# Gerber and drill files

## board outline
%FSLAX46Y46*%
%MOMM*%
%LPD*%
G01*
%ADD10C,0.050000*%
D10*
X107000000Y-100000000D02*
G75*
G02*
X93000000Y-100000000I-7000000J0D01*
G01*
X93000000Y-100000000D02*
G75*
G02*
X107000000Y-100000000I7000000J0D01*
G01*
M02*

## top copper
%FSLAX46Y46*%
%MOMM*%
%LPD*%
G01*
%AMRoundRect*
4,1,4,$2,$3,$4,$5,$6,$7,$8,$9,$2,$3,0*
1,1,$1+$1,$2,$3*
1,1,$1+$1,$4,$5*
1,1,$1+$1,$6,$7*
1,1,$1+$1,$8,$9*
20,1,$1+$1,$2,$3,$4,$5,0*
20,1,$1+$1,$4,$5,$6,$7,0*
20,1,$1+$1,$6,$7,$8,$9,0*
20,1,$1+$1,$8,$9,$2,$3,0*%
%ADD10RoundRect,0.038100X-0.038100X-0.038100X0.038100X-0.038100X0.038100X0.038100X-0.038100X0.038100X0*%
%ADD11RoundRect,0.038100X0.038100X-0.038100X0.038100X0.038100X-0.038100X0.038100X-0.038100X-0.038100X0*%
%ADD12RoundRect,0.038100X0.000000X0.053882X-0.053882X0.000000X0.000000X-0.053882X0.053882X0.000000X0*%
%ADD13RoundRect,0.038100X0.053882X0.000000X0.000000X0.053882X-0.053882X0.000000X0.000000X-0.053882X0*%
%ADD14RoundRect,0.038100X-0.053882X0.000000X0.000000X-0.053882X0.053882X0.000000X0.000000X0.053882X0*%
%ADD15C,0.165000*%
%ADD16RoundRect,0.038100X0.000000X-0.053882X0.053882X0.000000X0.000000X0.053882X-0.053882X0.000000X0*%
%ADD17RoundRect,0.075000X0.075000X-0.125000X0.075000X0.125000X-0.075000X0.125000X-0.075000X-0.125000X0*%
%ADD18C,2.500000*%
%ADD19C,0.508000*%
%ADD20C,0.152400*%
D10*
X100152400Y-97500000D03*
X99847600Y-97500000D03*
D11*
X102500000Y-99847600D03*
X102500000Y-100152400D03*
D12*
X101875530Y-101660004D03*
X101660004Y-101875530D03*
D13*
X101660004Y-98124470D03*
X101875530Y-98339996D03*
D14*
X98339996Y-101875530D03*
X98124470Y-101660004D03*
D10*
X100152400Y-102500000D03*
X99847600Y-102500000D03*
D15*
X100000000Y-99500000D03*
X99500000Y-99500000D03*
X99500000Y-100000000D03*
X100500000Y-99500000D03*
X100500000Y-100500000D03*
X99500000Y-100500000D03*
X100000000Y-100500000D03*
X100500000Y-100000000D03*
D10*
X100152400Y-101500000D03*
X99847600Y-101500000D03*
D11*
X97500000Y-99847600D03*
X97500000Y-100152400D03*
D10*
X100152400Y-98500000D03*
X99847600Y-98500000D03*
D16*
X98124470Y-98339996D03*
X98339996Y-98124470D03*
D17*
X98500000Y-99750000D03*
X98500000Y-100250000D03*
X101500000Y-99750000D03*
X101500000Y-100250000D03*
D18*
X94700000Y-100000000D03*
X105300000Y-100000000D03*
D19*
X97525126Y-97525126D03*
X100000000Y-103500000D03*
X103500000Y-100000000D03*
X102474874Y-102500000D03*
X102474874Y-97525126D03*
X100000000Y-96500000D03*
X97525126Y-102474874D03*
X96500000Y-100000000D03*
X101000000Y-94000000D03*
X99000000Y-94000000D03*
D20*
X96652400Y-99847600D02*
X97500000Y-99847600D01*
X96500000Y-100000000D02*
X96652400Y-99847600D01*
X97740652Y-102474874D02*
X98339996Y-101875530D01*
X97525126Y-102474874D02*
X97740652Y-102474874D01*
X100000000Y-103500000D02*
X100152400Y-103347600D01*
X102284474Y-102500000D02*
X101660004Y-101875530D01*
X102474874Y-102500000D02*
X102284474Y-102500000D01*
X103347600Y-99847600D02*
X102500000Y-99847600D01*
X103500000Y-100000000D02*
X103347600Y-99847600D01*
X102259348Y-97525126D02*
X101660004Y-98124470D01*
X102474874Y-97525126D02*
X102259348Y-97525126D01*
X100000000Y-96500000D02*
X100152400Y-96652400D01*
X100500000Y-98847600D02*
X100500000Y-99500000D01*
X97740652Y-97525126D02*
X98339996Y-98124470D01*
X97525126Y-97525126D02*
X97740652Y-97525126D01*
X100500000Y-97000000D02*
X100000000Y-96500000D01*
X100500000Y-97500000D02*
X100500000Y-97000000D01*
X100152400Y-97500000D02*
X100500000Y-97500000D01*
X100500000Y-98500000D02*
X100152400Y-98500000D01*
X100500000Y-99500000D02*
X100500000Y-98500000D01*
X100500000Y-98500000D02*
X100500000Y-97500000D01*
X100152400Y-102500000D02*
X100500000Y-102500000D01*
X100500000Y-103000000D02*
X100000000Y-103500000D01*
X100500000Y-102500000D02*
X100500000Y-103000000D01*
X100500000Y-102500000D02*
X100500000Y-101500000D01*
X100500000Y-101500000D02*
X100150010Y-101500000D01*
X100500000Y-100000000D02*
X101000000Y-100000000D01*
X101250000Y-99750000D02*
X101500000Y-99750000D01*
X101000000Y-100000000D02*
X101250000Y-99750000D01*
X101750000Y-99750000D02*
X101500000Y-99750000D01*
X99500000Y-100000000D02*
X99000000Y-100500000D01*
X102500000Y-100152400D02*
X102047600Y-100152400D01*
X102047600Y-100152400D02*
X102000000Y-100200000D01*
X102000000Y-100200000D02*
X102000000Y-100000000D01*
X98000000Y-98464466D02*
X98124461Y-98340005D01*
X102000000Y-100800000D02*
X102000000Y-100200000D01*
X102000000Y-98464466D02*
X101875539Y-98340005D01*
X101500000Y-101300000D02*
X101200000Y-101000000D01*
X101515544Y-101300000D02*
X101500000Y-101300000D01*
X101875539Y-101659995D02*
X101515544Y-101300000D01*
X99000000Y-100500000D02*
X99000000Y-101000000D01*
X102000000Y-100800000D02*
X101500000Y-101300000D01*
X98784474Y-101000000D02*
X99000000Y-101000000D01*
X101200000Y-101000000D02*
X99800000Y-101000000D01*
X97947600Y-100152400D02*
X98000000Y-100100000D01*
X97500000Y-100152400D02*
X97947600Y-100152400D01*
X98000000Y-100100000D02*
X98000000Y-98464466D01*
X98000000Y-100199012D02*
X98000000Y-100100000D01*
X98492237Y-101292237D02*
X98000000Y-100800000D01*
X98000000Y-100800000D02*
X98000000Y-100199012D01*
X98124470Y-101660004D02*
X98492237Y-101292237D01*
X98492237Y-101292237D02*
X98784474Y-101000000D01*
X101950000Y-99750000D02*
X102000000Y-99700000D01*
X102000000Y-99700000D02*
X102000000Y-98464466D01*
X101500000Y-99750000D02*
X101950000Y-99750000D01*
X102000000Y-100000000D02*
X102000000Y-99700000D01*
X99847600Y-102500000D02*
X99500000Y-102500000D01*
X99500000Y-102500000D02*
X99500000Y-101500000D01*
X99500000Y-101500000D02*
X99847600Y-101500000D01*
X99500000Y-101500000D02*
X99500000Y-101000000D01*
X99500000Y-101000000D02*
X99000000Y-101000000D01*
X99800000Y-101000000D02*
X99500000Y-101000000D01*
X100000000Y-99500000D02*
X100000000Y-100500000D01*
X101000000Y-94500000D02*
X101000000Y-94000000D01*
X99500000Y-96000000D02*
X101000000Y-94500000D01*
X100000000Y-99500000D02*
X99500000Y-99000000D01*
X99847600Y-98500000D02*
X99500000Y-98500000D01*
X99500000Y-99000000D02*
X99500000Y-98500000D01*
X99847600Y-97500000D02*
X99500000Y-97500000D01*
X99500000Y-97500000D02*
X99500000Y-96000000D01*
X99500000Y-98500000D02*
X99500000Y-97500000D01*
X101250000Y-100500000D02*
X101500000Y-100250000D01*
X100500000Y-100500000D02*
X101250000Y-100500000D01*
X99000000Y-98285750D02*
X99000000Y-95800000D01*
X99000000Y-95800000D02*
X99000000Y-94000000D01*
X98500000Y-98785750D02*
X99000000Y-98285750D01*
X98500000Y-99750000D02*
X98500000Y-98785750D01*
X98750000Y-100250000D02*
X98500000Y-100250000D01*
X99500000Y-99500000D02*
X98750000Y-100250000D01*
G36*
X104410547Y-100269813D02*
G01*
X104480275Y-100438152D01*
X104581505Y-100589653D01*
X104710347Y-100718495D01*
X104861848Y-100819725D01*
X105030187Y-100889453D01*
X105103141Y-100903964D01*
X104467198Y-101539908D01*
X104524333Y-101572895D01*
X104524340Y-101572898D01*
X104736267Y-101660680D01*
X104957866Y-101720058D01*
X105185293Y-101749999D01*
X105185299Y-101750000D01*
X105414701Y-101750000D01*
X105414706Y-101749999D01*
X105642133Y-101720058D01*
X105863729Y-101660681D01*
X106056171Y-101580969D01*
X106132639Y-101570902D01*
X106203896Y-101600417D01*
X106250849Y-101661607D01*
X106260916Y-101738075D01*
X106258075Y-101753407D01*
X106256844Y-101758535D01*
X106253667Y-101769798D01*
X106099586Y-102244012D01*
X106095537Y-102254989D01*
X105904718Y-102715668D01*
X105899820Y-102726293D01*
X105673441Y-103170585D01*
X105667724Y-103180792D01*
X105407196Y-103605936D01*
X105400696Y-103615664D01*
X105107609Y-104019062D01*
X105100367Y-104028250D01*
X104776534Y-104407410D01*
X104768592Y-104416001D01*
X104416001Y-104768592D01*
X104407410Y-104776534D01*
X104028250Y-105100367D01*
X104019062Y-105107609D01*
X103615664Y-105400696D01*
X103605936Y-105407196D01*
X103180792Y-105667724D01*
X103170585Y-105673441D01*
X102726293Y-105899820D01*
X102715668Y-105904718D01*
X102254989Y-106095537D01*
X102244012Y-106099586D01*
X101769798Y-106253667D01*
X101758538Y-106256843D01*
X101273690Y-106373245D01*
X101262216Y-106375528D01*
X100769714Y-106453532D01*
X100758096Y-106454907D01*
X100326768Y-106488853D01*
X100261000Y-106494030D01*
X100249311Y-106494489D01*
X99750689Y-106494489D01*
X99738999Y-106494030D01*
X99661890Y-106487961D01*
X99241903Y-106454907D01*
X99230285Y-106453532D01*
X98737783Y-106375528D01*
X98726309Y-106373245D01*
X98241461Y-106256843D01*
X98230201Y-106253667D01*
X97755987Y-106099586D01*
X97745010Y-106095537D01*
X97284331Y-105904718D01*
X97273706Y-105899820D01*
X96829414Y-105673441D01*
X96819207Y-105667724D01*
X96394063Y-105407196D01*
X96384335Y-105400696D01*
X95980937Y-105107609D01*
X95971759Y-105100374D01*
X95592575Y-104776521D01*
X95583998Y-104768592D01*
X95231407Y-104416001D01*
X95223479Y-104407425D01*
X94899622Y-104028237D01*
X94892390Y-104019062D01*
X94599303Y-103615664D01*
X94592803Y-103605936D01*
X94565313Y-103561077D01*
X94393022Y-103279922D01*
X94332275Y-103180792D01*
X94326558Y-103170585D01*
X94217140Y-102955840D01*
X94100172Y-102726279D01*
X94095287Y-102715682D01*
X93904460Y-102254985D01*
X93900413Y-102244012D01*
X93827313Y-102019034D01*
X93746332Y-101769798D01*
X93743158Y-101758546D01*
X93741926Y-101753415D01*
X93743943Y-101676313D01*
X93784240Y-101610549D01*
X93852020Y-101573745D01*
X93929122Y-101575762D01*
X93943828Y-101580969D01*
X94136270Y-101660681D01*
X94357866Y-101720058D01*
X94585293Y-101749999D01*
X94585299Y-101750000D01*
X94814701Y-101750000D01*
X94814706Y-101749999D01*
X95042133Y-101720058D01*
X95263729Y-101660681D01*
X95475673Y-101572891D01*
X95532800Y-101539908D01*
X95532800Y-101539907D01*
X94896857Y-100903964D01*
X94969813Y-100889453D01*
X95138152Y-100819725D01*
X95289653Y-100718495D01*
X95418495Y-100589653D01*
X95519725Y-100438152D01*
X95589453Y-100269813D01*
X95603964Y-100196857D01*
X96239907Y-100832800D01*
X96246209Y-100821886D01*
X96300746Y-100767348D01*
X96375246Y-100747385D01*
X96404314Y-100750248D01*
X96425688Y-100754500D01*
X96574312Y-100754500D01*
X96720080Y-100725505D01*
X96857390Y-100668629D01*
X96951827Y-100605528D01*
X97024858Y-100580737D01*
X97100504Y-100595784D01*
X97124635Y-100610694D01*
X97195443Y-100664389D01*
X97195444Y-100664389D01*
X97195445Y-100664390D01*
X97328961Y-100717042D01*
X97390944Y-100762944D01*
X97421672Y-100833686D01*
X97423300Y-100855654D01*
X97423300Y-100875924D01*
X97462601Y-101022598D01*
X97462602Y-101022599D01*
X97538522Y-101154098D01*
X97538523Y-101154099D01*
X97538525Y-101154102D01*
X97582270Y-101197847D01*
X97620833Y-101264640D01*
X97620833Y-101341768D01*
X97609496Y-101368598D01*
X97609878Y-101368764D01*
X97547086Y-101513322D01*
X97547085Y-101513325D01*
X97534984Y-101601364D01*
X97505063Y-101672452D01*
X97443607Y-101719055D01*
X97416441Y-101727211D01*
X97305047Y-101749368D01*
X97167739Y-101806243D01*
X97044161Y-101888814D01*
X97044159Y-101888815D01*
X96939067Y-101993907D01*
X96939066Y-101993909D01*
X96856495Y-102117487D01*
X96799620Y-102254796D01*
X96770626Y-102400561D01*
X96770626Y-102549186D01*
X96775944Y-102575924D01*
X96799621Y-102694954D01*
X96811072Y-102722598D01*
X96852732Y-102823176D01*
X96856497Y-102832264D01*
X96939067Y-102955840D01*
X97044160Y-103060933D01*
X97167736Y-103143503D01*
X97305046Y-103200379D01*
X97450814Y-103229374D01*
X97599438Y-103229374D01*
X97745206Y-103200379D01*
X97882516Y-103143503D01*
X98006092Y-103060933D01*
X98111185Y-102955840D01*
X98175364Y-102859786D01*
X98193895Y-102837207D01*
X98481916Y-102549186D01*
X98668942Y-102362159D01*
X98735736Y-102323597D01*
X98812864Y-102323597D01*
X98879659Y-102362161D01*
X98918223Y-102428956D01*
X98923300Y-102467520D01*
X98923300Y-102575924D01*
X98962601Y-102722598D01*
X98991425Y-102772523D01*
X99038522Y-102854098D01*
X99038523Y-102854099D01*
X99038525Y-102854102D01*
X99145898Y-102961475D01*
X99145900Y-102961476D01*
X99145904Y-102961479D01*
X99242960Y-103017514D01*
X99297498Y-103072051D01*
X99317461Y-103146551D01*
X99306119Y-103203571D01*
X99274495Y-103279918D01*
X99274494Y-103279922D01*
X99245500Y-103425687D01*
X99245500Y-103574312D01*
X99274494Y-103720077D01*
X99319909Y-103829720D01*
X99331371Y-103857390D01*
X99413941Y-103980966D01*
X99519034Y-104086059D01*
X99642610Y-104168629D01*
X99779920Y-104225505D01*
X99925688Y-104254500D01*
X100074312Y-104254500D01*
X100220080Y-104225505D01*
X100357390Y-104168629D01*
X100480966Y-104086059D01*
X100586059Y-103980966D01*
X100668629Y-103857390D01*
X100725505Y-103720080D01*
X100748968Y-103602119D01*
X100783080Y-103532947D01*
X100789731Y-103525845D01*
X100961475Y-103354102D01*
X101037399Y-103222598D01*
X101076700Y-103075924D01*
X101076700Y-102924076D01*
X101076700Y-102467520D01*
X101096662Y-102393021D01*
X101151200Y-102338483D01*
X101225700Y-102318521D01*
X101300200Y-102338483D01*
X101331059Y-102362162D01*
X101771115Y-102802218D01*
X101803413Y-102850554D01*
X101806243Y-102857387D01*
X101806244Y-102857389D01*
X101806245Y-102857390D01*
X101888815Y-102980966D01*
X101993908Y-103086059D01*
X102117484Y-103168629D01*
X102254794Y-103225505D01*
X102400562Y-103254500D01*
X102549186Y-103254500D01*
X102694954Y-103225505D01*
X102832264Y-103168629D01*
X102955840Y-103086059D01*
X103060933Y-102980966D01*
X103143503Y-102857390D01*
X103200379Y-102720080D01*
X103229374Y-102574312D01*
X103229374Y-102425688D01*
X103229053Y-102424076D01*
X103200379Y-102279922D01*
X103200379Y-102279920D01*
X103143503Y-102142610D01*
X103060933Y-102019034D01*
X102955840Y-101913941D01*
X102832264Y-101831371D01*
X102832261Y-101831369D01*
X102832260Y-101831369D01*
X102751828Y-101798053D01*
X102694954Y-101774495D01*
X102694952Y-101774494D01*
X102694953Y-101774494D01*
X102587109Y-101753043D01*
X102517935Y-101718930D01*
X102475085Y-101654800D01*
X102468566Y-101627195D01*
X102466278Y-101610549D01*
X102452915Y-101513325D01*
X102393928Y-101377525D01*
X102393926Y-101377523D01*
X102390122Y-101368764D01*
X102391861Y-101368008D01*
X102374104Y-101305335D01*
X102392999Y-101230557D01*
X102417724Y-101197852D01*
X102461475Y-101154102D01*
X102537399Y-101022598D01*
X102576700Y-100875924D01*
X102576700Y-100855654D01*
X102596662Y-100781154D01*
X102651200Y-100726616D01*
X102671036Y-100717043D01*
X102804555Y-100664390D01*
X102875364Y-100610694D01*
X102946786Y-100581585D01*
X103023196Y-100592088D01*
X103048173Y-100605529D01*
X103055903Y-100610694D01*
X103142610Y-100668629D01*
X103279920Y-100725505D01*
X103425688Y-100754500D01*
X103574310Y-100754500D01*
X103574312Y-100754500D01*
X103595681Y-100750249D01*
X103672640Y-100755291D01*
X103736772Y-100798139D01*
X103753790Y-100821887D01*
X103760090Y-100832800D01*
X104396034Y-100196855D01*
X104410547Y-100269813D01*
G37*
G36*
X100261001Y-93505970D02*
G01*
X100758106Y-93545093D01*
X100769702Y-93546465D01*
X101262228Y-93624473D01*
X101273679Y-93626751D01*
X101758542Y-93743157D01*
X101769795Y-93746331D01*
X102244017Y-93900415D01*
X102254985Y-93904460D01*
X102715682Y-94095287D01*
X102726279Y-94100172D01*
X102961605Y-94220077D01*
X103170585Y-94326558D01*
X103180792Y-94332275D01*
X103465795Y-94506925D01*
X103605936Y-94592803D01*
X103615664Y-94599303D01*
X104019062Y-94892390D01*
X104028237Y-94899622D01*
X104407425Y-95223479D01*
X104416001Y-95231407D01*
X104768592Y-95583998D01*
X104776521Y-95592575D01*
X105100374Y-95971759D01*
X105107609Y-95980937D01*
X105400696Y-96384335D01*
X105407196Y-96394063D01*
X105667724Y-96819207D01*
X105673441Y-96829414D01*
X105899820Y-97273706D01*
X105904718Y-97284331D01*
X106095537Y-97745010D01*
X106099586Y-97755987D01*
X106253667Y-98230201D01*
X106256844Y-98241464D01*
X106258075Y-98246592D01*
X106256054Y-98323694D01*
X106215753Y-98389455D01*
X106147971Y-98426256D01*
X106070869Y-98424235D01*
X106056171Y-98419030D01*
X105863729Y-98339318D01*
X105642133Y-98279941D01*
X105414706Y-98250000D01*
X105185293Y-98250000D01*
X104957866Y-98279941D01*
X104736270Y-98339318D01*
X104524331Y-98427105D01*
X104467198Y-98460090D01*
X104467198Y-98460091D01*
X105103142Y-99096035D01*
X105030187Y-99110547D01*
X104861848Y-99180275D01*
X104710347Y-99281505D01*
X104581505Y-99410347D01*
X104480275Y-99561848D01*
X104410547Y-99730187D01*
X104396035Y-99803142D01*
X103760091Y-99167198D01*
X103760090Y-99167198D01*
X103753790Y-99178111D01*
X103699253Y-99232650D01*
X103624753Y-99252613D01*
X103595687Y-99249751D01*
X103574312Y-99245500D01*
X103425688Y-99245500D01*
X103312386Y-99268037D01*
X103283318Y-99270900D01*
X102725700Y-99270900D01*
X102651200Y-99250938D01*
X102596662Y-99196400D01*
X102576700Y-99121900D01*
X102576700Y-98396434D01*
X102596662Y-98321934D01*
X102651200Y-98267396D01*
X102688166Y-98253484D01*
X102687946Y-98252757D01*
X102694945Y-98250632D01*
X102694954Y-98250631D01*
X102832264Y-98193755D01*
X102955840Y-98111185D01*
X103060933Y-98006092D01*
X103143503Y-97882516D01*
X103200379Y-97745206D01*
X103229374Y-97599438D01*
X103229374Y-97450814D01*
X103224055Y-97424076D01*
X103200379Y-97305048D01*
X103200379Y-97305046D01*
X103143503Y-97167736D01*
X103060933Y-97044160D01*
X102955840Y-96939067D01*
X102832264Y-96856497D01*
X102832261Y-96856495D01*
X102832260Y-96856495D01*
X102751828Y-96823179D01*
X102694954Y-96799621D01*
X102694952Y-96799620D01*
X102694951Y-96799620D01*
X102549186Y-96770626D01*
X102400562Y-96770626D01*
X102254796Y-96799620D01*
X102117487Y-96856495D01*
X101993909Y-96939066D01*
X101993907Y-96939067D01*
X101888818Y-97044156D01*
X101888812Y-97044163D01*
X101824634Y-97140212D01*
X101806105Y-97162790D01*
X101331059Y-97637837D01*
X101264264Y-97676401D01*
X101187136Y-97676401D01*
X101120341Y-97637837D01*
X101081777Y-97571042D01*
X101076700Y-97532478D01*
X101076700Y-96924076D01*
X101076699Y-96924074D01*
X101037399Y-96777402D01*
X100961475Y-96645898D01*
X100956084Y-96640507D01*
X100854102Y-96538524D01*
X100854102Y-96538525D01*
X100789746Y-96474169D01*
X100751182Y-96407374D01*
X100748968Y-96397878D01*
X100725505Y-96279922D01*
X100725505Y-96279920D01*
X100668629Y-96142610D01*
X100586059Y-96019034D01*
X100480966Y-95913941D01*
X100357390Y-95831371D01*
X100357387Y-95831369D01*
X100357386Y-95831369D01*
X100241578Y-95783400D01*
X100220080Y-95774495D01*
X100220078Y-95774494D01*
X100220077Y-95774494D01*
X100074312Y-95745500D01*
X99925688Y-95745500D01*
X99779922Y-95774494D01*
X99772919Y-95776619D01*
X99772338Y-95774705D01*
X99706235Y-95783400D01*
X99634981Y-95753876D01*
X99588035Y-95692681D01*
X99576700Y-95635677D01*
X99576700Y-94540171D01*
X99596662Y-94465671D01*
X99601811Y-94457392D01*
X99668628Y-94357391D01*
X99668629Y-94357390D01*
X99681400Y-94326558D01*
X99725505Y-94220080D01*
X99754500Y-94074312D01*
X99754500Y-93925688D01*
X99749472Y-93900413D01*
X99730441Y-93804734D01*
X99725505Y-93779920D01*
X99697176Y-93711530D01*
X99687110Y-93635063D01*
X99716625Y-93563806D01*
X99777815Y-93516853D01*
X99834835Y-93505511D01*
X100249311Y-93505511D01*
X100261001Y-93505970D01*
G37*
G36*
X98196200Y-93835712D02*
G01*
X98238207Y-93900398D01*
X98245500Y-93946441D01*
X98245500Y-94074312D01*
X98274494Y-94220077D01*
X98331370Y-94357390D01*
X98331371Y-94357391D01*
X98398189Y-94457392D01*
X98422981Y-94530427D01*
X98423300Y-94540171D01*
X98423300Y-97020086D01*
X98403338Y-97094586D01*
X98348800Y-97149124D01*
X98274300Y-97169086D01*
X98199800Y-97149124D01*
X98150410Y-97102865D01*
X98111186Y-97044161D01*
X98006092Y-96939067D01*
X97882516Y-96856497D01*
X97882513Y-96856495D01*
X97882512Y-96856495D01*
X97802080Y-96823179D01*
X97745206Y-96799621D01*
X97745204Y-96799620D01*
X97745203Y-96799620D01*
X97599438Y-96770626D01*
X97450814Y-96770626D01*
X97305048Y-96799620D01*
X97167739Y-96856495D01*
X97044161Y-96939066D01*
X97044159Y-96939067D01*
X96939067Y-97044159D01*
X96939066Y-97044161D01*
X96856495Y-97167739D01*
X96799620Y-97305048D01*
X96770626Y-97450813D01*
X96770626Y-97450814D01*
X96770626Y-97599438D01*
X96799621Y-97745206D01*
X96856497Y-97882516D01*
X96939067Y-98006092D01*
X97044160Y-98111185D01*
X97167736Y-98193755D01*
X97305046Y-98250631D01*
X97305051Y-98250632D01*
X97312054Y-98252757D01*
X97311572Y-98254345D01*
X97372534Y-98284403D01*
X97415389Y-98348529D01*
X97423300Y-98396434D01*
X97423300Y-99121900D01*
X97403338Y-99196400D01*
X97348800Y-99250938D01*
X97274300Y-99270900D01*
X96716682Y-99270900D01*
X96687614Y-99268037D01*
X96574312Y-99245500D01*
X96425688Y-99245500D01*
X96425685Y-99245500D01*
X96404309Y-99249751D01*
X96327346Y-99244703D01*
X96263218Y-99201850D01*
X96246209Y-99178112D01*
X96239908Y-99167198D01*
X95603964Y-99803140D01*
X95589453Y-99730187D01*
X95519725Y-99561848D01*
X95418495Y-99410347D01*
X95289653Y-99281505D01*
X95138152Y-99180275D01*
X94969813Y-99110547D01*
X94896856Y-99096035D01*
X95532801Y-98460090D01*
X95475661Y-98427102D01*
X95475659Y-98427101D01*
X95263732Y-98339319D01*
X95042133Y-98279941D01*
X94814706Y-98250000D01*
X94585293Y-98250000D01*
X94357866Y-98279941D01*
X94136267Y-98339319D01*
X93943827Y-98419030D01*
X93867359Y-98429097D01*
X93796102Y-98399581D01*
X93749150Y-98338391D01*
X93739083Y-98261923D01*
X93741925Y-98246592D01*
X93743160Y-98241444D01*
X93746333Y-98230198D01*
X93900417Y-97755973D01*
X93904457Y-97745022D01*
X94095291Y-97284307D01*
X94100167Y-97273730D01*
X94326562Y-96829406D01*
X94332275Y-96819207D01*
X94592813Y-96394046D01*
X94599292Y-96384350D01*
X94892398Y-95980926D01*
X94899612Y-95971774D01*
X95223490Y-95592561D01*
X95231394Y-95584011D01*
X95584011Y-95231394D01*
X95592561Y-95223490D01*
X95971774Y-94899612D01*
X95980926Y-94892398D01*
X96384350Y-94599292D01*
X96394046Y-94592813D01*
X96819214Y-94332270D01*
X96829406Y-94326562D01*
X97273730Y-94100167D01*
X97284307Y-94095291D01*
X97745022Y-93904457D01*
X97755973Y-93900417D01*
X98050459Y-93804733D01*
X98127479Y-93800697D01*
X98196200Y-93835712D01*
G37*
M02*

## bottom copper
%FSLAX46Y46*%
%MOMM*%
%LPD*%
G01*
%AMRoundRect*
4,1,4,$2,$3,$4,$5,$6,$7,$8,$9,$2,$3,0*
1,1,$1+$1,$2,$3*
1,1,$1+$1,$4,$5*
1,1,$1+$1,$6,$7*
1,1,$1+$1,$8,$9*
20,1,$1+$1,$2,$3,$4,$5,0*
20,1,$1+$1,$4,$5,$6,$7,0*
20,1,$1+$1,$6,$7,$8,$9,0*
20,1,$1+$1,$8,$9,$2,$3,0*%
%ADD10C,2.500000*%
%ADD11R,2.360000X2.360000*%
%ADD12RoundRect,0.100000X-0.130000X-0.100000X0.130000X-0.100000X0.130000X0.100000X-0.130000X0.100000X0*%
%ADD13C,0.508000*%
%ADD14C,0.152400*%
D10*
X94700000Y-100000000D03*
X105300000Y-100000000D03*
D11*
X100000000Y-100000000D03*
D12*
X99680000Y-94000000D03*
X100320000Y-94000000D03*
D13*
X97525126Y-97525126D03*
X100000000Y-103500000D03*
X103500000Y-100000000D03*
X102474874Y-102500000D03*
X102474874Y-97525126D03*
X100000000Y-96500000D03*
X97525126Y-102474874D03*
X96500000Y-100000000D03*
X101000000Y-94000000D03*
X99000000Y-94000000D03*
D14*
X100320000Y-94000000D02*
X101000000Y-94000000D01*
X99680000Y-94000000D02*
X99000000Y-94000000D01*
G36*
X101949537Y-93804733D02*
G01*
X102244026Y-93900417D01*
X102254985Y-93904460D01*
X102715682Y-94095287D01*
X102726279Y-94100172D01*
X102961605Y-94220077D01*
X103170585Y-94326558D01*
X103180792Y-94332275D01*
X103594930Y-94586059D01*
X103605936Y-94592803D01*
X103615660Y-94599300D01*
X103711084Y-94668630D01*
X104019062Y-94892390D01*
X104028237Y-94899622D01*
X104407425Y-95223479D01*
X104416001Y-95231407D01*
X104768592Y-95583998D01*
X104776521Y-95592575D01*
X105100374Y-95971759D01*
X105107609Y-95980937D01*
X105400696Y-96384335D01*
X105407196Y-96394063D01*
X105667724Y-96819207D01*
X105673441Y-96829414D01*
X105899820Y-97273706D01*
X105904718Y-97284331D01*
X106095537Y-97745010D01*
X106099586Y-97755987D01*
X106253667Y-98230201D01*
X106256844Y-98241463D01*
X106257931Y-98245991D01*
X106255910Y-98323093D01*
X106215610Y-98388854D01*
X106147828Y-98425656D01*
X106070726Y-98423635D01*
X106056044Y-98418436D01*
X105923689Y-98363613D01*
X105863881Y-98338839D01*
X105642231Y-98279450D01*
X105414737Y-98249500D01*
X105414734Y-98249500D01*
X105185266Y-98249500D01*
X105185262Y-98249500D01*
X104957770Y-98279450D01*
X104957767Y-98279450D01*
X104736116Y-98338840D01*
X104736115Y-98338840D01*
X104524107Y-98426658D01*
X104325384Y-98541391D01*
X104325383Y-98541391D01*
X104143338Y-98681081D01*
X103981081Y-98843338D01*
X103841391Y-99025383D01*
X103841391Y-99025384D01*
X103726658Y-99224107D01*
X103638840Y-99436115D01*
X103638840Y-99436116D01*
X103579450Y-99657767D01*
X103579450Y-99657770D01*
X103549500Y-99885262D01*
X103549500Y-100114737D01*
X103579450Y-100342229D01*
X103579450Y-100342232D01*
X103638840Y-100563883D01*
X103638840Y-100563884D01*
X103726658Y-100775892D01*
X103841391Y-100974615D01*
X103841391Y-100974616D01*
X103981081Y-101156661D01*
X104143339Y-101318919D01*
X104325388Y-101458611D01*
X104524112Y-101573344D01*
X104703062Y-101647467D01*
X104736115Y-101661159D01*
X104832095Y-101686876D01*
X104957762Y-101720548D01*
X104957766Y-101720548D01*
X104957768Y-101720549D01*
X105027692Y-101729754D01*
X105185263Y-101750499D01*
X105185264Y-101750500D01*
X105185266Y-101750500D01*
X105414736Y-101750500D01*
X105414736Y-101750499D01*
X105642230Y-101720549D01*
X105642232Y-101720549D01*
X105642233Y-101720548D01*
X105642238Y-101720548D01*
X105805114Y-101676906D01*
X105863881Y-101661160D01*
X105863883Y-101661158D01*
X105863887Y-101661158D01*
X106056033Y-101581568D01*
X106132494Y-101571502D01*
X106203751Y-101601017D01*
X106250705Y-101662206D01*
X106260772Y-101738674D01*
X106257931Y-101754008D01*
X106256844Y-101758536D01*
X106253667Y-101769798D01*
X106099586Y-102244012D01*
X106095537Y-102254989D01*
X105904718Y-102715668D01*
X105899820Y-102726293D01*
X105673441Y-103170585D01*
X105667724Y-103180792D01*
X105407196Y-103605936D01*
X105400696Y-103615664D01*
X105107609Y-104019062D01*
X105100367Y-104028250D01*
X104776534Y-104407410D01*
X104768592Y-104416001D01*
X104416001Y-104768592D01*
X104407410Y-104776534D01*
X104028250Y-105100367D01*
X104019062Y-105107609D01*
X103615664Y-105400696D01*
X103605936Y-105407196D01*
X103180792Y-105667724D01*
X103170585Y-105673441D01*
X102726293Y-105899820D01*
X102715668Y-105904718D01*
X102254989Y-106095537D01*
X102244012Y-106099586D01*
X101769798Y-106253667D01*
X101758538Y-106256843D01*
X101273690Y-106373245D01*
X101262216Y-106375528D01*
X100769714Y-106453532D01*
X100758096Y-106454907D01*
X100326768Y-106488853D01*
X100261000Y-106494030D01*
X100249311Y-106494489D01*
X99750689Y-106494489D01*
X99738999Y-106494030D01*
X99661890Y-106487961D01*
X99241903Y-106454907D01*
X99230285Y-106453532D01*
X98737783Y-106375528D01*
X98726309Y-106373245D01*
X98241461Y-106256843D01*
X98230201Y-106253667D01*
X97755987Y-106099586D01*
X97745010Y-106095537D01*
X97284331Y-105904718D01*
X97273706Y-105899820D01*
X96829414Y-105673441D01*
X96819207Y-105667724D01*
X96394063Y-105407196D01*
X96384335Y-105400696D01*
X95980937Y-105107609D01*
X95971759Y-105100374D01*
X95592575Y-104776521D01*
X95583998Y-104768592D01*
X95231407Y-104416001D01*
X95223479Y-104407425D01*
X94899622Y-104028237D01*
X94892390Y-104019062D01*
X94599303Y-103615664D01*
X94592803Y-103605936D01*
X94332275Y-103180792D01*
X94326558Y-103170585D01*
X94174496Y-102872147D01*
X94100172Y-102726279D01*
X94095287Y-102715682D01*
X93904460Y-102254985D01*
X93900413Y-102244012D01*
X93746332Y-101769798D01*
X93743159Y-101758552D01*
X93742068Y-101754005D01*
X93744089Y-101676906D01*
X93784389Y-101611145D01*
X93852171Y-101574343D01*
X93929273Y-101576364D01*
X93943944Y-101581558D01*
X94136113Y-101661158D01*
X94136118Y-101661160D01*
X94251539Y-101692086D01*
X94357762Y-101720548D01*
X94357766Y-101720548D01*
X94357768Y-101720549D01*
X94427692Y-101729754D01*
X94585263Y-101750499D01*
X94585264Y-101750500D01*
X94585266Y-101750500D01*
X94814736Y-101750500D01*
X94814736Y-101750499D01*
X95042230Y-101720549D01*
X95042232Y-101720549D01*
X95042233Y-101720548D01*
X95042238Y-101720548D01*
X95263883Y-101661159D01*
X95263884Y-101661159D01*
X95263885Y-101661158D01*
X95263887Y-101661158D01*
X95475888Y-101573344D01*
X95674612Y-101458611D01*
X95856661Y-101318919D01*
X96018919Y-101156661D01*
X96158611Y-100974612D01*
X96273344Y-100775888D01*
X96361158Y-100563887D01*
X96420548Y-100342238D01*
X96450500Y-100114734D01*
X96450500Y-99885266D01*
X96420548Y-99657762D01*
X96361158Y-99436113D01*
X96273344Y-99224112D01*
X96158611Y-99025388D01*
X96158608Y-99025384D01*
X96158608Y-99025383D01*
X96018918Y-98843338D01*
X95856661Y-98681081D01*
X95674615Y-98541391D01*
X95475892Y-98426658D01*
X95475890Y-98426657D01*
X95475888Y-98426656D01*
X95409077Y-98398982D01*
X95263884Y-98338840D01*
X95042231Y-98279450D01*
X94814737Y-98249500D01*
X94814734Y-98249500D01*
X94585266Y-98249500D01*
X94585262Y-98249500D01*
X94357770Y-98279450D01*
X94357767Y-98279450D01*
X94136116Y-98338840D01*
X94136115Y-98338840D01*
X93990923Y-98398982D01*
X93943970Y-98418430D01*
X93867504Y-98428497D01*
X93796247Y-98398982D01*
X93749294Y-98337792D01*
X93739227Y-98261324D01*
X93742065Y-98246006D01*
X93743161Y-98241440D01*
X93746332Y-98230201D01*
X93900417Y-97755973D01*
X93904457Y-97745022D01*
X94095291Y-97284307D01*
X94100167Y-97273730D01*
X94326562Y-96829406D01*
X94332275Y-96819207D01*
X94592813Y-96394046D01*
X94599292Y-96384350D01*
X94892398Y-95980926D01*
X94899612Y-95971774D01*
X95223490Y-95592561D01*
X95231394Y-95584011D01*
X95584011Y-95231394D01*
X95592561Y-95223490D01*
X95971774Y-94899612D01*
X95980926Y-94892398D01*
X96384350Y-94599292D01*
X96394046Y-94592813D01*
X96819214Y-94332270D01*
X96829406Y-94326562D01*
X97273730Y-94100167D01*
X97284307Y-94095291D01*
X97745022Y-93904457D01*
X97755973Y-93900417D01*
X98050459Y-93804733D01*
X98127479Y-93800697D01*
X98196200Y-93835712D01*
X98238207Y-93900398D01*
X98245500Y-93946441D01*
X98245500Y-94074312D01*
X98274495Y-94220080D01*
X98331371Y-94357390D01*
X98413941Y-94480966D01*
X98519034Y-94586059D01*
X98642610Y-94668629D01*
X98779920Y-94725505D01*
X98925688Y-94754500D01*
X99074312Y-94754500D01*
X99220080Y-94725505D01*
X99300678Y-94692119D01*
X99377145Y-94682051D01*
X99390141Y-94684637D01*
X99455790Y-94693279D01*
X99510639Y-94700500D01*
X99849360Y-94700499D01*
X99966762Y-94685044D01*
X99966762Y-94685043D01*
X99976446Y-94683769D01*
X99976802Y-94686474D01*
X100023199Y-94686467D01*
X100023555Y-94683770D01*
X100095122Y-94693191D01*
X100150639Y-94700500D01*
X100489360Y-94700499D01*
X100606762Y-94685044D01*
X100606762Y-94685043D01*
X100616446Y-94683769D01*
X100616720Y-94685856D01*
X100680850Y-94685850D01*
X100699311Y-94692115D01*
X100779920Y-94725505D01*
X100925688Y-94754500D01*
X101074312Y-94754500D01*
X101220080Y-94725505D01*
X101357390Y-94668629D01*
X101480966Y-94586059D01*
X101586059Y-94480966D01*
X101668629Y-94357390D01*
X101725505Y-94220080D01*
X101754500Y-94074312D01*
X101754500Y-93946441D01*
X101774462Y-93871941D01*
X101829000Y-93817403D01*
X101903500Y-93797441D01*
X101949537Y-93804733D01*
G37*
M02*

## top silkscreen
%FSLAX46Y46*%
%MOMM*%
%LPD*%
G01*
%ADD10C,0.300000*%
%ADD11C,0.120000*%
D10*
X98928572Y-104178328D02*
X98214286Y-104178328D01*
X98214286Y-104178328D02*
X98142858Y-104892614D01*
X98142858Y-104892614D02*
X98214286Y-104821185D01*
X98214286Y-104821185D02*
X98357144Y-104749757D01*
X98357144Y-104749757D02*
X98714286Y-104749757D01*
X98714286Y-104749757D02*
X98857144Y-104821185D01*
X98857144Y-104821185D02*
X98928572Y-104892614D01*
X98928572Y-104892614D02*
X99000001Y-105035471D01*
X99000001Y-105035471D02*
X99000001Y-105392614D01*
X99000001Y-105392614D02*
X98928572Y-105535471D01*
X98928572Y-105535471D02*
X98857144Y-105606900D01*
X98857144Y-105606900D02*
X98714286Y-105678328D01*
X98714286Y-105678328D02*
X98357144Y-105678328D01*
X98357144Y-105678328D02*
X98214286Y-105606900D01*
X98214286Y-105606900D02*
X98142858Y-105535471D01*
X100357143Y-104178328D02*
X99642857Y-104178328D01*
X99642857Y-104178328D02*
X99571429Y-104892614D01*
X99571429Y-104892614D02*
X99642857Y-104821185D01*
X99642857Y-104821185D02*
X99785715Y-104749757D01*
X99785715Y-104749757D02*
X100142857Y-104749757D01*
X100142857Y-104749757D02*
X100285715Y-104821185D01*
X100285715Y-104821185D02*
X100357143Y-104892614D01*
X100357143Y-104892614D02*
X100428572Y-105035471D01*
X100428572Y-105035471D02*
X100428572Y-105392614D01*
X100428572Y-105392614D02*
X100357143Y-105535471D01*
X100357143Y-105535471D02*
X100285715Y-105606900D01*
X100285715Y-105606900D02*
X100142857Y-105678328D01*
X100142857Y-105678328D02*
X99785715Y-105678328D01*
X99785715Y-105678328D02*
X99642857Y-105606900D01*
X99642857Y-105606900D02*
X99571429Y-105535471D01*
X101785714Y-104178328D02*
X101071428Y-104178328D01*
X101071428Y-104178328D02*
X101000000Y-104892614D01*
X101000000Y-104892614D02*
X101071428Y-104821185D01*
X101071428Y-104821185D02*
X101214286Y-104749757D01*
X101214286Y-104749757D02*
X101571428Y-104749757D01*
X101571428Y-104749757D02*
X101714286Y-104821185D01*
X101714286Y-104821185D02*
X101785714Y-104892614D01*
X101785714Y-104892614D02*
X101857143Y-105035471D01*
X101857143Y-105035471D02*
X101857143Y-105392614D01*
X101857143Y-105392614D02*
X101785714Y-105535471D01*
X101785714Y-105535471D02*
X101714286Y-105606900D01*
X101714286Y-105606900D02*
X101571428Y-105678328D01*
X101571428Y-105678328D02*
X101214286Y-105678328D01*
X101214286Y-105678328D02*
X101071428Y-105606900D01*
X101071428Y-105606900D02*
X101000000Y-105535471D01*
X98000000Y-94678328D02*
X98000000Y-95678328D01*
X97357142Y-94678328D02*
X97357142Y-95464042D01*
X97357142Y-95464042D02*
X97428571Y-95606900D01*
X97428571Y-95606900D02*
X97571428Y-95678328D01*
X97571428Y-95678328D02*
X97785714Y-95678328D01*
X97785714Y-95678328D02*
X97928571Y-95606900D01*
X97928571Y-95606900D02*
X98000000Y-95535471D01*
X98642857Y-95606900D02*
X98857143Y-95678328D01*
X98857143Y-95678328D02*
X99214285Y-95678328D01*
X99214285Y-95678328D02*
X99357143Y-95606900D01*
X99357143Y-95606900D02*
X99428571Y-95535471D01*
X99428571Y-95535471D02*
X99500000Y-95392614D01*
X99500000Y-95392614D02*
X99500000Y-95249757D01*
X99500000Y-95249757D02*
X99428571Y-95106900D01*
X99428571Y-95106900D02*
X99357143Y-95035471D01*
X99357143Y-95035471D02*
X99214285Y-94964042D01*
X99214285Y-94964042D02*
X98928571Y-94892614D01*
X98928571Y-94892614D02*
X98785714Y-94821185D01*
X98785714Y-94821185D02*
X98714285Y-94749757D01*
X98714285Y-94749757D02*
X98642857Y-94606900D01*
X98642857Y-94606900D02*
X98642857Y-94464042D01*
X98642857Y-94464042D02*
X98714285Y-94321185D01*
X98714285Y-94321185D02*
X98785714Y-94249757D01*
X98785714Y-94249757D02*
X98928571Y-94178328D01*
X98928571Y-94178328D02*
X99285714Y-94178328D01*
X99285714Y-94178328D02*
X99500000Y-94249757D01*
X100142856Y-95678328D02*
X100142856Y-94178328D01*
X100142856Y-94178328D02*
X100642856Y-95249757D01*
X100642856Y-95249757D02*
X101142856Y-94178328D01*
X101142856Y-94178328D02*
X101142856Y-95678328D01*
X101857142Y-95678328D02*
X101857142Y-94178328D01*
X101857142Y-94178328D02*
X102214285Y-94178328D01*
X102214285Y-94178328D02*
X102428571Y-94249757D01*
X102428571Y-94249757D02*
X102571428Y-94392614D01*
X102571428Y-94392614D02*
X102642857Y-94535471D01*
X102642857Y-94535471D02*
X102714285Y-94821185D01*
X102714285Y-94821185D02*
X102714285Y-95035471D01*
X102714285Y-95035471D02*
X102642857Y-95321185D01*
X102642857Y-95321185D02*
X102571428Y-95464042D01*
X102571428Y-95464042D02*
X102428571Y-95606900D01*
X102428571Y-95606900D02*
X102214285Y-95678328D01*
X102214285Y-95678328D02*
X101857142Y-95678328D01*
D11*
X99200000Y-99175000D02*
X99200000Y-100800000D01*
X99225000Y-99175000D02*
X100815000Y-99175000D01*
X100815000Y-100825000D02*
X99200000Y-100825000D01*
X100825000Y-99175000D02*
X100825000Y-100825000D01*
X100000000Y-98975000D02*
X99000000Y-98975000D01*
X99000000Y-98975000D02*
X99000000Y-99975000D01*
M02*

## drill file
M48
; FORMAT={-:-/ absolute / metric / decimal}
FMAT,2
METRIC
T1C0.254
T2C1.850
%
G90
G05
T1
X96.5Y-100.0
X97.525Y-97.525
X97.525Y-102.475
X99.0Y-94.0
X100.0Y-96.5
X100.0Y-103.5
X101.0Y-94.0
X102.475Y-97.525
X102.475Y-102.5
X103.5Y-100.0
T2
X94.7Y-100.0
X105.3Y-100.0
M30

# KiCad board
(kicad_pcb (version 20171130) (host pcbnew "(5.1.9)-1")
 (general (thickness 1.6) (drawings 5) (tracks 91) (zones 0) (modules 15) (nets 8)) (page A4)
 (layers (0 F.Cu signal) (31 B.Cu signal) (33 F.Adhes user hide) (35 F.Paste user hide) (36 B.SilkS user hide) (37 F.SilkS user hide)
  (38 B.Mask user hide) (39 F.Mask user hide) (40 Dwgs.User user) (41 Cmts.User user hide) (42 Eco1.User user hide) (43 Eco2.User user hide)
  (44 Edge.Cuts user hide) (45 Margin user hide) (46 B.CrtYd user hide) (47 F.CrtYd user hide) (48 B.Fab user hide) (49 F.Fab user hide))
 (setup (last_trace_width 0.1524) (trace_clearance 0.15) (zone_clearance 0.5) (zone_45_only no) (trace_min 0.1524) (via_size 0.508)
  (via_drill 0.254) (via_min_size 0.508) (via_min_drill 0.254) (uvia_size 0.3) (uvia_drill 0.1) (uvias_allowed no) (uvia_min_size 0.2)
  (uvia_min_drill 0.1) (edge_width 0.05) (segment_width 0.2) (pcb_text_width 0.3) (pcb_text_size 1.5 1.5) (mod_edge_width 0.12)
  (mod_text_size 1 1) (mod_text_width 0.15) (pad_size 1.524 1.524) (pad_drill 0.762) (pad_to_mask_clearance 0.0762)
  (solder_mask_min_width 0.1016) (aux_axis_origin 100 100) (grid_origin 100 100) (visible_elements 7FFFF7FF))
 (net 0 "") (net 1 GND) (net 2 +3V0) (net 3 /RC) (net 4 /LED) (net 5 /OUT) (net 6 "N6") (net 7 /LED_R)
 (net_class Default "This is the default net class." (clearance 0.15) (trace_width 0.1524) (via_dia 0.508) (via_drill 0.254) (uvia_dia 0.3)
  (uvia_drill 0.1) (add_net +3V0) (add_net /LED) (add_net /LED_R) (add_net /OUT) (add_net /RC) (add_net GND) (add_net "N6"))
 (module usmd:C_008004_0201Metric (layer F.Cu) (at 100 97.5)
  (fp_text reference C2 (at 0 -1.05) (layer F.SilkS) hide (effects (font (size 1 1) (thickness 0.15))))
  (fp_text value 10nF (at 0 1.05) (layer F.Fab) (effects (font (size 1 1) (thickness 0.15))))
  (pad 2 smd roundrect (at 0.1524 0) (size 0.1524 0.1524) (layers F.Cu F.Mask) (roundrect_rratio 0.25) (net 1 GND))
  (pad 1 smd roundrect (at -0.1524 0) (size 0.1524 0.1524) (layers F.Cu F.Paste F.Mask) (roundrect_rratio 0.25) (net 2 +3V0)))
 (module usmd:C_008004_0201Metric (layer F.Cu) (at 102.5 100 90)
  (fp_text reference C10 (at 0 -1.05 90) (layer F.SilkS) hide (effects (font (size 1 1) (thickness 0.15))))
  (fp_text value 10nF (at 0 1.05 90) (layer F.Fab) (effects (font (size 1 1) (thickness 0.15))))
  (pad 2 smd roundrect (at 0.1524 0 90) (size 0.1524 0.1524) (layers F.Cu F.Mask) (roundrect_rratio 0.25) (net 1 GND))
  (pad 1 smd roundrect (at -0.1524 0 90) (size 0.1524 0.1524) (layers F.Cu F.Paste F.Mask) (roundrect_rratio 0.25) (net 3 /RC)))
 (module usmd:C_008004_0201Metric (layer F.Cu) (at 101.767767 101.767767 225)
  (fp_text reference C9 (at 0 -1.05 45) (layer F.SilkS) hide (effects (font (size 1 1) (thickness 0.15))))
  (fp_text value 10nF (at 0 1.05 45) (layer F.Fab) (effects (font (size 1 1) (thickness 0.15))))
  (pad 1 smd roundrect (at -0.1524 0 225) (size 0.1524 0.1524) (layers F.Cu F.Paste F.Mask) (roundrect_rratio 0.25) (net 3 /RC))
  (pad 2 smd roundrect (at 0.1524 0 225) (size 0.1524 0.1524) (layers F.Cu F.Mask) (roundrect_rratio 0.25) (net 1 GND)))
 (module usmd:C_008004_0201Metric (layer F.Cu) (at 101.767767 98.232233 135)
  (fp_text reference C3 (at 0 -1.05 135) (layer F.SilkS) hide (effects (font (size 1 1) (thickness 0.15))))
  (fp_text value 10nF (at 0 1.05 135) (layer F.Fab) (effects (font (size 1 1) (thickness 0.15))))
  (pad 2 smd roundrect (at 0.1524 0 135) (size 0.1524 0.1524) (layers F.Cu F.Mask) (roundrect_rratio 0.25) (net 1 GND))
  (pad 1 smd roundrect (at -0.1524 0 135) (size 0.1524 0.1524) (layers F.Cu F.Paste F.Mask) (roundrect_rratio 0.25) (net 3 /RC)))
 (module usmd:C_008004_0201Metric (layer F.Cu) (at 98.232233 101.767767 315)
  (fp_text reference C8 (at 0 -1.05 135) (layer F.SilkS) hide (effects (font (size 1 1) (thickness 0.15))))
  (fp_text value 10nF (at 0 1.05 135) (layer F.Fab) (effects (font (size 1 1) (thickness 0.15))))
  (pad 2 smd roundrect (at 0.1524 0 315) (size 0.1524 0.1524) (layers F.Cu F.Mask) (roundrect_rratio 0.25) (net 1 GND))
  (pad 1 smd roundrect (at -0.1524 0 315) (size 0.1524 0.1524) (layers F.Cu F.Paste F.Mask) (roundrect_rratio 0.25) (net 3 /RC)))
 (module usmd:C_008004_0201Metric (layer F.Cu) (at 100 102.5)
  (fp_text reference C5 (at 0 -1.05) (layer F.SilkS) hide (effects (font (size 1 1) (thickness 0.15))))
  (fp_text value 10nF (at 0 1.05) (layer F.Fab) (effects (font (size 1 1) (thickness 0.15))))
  (pad 2 smd roundrect (at 0.1524 0) (size 0.1524 0.1524) (layers F.Cu F.Mask) (roundrect_rratio 0.25) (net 1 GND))
  (pad 1 smd roundrect (at -0.1524 0) (size 0.1524 0.1524) (layers F.Cu F.Paste F.Mask) (roundrect_rratio 0.25) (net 3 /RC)))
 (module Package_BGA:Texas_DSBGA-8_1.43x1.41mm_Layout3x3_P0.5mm (layer F.Cu) (at 100 100) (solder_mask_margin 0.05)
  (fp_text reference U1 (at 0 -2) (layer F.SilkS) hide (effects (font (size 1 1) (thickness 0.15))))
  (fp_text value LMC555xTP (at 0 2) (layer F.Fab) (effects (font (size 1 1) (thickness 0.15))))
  (fp_line (start -0.8 -0.825) (end -0.8 0.8) (layer F.SilkS) (width 0.12))
  (fp_line (start -0.775 -0.825) (end 0.815 -0.825) (layer F.SilkS) (width 0.12))
  (fp_line (start 0.815 0.825) (end -0.8 0.825) (layer F.SilkS) (width 0.12))
  (fp_line (start 0.825 -0.825) (end 0.825 0.825) (layer F.SilkS) (width 0.12))
  (fp_line (start 0 -1.025) (end -1 -1.025) (layer F.SilkS) (width 0.12))
  (fp_line (start -1 -1.025) (end -1 -0.025) (layer F.SilkS) (width 0.12))
  (pad "" smd rect (at 0.5 0.5) (size 0.3 0.3) (layers F.Paste)) (pad "" smd rect (at 0 0.5) (size 0.3 0.3) (layers F.Paste))
  (pad "" smd rect (at -0.5 0.5) (size 0.3 0.3) (layers F.Paste)) (pad "" smd rect (at 0.5 0) (size 0.3 0.3) (layers F.Paste))
  (pad "" smd rect (at -0.5 0) (size 0.3 0.3) (layers F.Paste))
  (pad "" smd rect (at 0.5 -0.5) (size 0.3 0.3) (layers F.Paste))
  (pad "" smd rect (at 0 -0.5) (size 0.3 0.3) (layers F.Paste))
  (pad "" smd rect (at -0.5 -0.5) (size 0.3 0.3) (layers F.Paste))
  (pad A2 smd circle (at 0 -0.5) (size 0.165 0.165) (layers F.Cu F.Mask) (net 2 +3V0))
  (pad A1 smd circle (at -0.5 -0.5) (size 0.165 0.165) (layers F.Cu F.Mask) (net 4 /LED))
  (pad B1 smd circle (at -0.5 0) (size 0.165 0.165) (layers F.Cu F.Mask) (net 3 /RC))
  (pad A3 smd circle (at 0.5 -0.5) (size 0.165 0.165) (layers F.Cu F.Mask) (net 1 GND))
  (pad C3 smd circle (at 0.5 0.5) (size 0.165 0.165) (layers F.Cu F.Mask) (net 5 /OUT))
  (pad C1 smd circle (at -0.5 0.5) (size 0.165 0.165) (layers F.Cu F.Mask) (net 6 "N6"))
  (pad C2 smd circle (at 0 0.5) (size 0.165 0.165) (layers F.Cu F.Mask) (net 2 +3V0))
  (pad B3 smd circle (at 0.5 0) (size 0.165 0.165) (layers F.Cu F.Paste F.Mask) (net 3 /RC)))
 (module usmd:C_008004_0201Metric (layer F.Cu) (at 100 101.5)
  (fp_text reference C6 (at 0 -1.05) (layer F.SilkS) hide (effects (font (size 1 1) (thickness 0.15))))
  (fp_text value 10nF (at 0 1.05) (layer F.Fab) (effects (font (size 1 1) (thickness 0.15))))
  (pad 2 smd roundrect (at 0.1524 0) (size 0.1524 0.1524) (layers F.Cu F.Mask) (roundrect_rratio 0.25) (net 1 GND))
  (pad 1 smd roundrect (at -0.1524 0) (size 0.1524 0.1524) (layers F.Cu F.Paste F.Mask) (roundrect_rratio 0.25) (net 3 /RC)))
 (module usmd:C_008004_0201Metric (layer F.Cu) (at 97.5 100 90)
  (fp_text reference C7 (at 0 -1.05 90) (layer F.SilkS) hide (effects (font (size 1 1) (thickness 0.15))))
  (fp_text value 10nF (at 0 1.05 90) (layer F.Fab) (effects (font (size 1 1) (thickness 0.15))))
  (pad 2 smd roundrect (at 0.1524 0 90) (size 0.1524 0.1524) (layers F.Cu F.Mask) (roundrect_rratio 0.25) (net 1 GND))
  (pad 1 smd roundrect (at -0.1524 0 90) (size 0.1524 0.1524) (layers F.Cu F.Paste F.Mask) (roundrect_rratio 0.25) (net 3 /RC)))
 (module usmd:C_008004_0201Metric (layer F.Cu) (at 100 98.5)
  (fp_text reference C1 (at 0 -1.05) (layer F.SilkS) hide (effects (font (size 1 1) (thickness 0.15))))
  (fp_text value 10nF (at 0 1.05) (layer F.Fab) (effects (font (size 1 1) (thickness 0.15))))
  (pad 2 smd roundrect (at 0.1524 0) (size 0.1524 0.1524) (layers F.Cu F.Mask) (roundrect_rratio 0.25) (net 1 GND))
  (pad 1 smd roundrect (at -0.1524 0) (size 0.1524 0.1524) (layers F.Cu F.Paste F.Mask) (roundrect_rratio 0.25) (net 2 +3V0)))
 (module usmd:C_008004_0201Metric (layer F.Cu) (at 98.232233 98.232233 45)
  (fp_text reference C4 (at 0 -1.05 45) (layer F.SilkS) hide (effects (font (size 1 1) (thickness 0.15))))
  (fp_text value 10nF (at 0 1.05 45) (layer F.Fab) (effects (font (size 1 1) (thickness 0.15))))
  (pad 1 smd roundrect (at -0.1524 0 45) (size 0.1524 0.1524) (layers F.Cu F.Paste F.Mask) (roundrect_rratio 0.25) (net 3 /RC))
  (pad 2 smd roundrect (at 0.1524 0 45) (size 0.1524 0.1524) (layers F.Cu F.Mask) (roundrect_rratio 0.25) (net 1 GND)))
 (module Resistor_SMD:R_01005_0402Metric (layer F.Cu) (at 98.5 100 90)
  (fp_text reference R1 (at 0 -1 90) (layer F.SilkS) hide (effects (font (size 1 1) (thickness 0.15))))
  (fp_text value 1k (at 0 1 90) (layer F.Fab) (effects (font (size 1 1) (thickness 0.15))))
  (pad 2 smd roundrect (at 0.25 0 90) (size 0.4 0.3) (layers F.Cu F.Mask) (roundrect_rratio 0.25) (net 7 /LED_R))
  (pad 1 smd roundrect (at -0.25 0 90) (size 0.4 0.3) (layers F.Cu F.Mask) (roundrect_rratio 0.25) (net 4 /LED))
  (pad "" smd roundrect (at 0.275 0 90) (size 0.27 0.27) (layers F.Paste) (roundrect_rratio 0.25))
  (pad "" smd roundrect (at -0.275 0 90) (size 0.27 0.27) (layers F.Paste) (roundrect_rratio 0.25)))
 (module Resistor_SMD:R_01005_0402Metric (layer F.Cu) (at 101.5 100 90)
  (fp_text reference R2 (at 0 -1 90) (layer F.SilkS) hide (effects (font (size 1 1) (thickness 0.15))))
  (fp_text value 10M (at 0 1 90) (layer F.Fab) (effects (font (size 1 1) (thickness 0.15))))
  (pad 2 smd roundrect (at 0.25 0 90) (size 0.4 0.3) (layers F.Cu F.Mask) (roundrect_rratio 0.25) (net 3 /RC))
  (pad 1 smd roundrect (at -0.25 0 90) (size 0.4 0.3) (layers F.Cu F.Mask) (roundrect_rratio 0.25) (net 5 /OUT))
  (pad "" smd roundrect (at 0.275 0 90) (size 0.27 0.27) (layers F.Paste) (roundrect_rratio 0.25))
  (pad "" smd roundrect (at -0.275 0 90) (size 0.27 0.27) (layers F.Paste) (roundrect_rratio 0.25)))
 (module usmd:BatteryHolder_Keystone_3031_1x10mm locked (layer B.Cu) (at 100 100)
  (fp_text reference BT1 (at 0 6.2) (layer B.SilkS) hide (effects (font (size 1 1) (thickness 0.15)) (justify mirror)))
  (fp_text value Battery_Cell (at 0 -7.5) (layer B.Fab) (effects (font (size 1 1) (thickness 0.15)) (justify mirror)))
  (pad 1 thru_hole circle (at -5.3 0) (size 2.5 2.5) (drill 1.85) (layers *.Cu *.Mask) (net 2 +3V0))
  (pad 1 thru_hole circle (at 5.3 0) (size 2.5 2.5) (drill 1.85) (layers *.Cu *.Mask) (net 2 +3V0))
  (pad 2 smd rect (at 0 0) (size 2.36 2.36) (layers B.Cu B.Mask) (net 1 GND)))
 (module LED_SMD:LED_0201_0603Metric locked (layer B.Cu) (at 100 94)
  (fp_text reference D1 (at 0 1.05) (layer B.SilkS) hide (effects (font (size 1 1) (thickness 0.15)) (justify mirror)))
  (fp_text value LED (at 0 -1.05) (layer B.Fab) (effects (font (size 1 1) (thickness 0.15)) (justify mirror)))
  (pad "" smd roundrect (at -0.345 0) (size 0.318 0.36) (layers B.Paste) (roundrect_rratio 0.25))
  (pad "" smd roundrect (at 0.345 0) (size 0.318 0.36) (layers B.Paste) (roundrect_rratio 0.25))
  (pad 1 smd roundrect (at -0.32 0) (size 0.46 0.4) (layers B.Cu B.Mask) (roundrect_rratio 0.25) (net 7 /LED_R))
  (pad 2 smd roundrect (at 0.32 0) (size 0.46 0.4) (layers B.Cu B.Mask) (roundrect_rratio 0.25) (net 2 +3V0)))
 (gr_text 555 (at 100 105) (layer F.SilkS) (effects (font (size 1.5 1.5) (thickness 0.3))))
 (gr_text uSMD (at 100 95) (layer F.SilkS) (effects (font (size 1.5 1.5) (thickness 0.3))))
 (gr_circle (center 100 100) (end 107 100) (layer Edge.Cuts) (width 0.05))
 (via (at 97.525126 97.525126) (size 0.508) (drill 0.254) (layers F.Cu B.Cu) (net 1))
 (via (at 100 103.5) (size 0.508) (drill 0.254) (layers F.Cu B.Cu) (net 1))
 (via (at 103.5 100) (size 0.508) (drill 0.254) (layers F.Cu B.Cu) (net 1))
 (via (at 102.474874 102.5) (size 0.508) (drill 0.254) (layers F.Cu B.Cu) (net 1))
 (via (at 102.474874 97.525126) (size 0.508) (drill 0.254) (layers F.Cu B.Cu) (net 1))
 (via (at 100 96.5) (size 0.508) (drill 0.254) (layers F.Cu B.Cu) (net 1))
 (via (at 97.525126 102.474874) (size 0.508) (drill 0.254) (layers F.Cu B.Cu) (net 1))
 (via (at 96.5 100) (size 0.508) (drill 0.254) (layers F.Cu B.Cu) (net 1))
 (segment (start 96.6524 99.8476) (end 97.5 99.8476) (width 0.1524) (layer F.Cu) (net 1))
 (segment (start 96.5 100) (end 96.6524 99.8476) (width 0.1524) (layer F.Cu) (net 1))
 (segment (start 97.740652 102.474874) (end 98.339996 101.87553) (width 0.1524) (layer F.Cu) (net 1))
 (segment (start 97.525126 102.474874) (end 97.740652 102.474874) (width 0.1524) (layer F.Cu) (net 1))
 (segment (start 100 103.5) (end 100.1524 103.3476) (width 0.1524) (layer F.Cu) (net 1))
 (segment (start 102.284474 102.5) (end 101.660004 101.87553) (width 0.1524) (layer F.Cu) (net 1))
 (segment (start 102.474874 102.5) (end 102.284474 102.5) (width 0.1524) (layer F.Cu) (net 1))
 (segment (start 103.3476 99.8476) (end 102.5 99.8476) (width 0.1524) (layer F.Cu) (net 1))
 (segment (start 103.5 100) (end 103.3476 99.8476) (width 0.1524) (layer F.Cu) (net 1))
 (segment (start 102.259348 97.525126) (end 101.660004 98.12447) (width 0.1524) (layer F.Cu) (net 1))
 (segment (start 102.474874 97.525126) (end 102.259348 97.525126) (width 0.1524) (layer F.Cu) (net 1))
 (segment (start 100 96.5) (end 100.1524 96.6524) (width 0.1524) (layer F.Cu) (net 1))
 (segment (start 100.5 98.8476) (end 100.5 99.5) (width 0.1524) (layer F.Cu) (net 1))
 (segment (start 97.740652 97.525126) (end 98.339996 98.12447) (width 0.1524) (layer F.Cu) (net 1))
 (segment (start 97.525126 97.525126) (end 97.740652 97.525126) (width 0.1524) (layer F.Cu) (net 1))
 (segment (start 100.5 97) (end 100 96.5) (width 0.1524) (layer F.Cu) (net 1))
 (segment (start 100.5 97.5) (end 100.5 97) (width 0.1524) (layer F.Cu) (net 1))
 (segment (start 100.1524 97.5) (end 100.5 97.5) (width 0.1524) (layer F.Cu) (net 1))
 (segment (start 100.5 98.5) (end 100.1524 98.5) (width 0.1524) (layer F.Cu) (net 1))
 (segment (start 100.5 99.5) (end 100.5 98.5) (width 0.1524) (layer F.Cu) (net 1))
 (segment (start 100.5 98.5) (end 100.5 97.5) (width 0.1524) (layer F.Cu) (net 1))
 (segment (start 100.1524 102.5) (end 100.5 102.5) (width 0.1524) (layer F.Cu) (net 1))
 (segment (start 100.5 103) (end 100 103.5) (width 0.1524) (layer F.Cu) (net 1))
 (segment (start 100.5 102.5) (end 100.5 103) (width 0.1524) (layer F.Cu) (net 1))
 (segment (start 100.5 102.5) (end 100.5 101.5) (width 0.1524) (layer F.Cu) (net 1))
 (segment (start 100.5 101.5) (end 100.15001 101.5) (width 0.1524) (layer F.Cu) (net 1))
 (segment (start 100.5 100) (end 101 100) (width 0.1524) (layer F.Cu) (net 3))
 (segment (start 101.25 99.75) (end 101.5 99.75) (width 0.1524) (layer F.Cu) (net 3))
 (segment (start 101 100) (end 101.25 99.75) (width 0.1524) (layer F.Cu) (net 3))
 (segment (start 101.75 99.75) (end 101.5 99.75) (width 0.1524) (layer F.Cu) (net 3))
 (segment (start 99.5 100) (end 99 100.5) (width 0.1524) (layer F.Cu) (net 3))
 (segment (start 102.5 100.1524) (end 102.0476 100.1524) (width 0.1524) (layer F.Cu) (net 3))
 (segment (start 102.0476 100.1524) (end 102 100.2) (width 0.1524) (layer F.Cu) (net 3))
 (segment (start 102 100.2) (end 102 100) (width 0.1524) (layer F.Cu) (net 3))
 (segment (start 98 98.464466) (end 98.124461 98.340005) (width 0.1524) (layer F.Cu) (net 3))
 (segment (start 102 100.8) (end 102 100.2) (width 0.1524) (layer F.Cu) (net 3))
 (segment (start 102 98.464466) (end 101.875539 98.340005) (width 0.1524) (layer F.Cu) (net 3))
 (segment (start 101.5 101.3) (end 101.2 101) (width 0.1524) (layer F.Cu) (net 3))
 (segment (start 101.515544 101.3) (end 101.5 101.3) (width 0.1524) (layer F.Cu) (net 3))
 (segment (start 101.875539 101.659995) (end 101.515544 101.3) (width 0.1524) (layer F.Cu) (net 3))
 (segment (start 99 100.5) (end 99 101) (width 0.1524) (layer F.Cu) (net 3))
 (segment (start 102 100.8) (end 101.5 101.3) (width 0.1524) (layer F.Cu) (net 3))
 (segment (start 98.784474 101) (end 99 101) (width 0.1524) (layer F.Cu) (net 3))
 (segment (start 101.2 101) (end 99.8 101) (width 0.1524) (layer F.Cu) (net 3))
 (segment (start 97.9476 100.1524) (end 98 100.1) (width 0.1524) (layer F.Cu) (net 3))
 (segment (start 97.5 100.1524) (end 97.9476 100.1524) (width 0.1524) (layer F.Cu) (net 3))
 (segment (start 98 100.1) (end 98 98.464466) (width 0.1524) (layer F.Cu) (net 3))
 (segment (start 98 100.199012) (end 98 100.1) (width 0.1524) (layer F.Cu) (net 3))
 (segment (start 98.492237 101.292237) (end 98 100.8) (width 0.1524) (layer F.Cu) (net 3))
 (segment (start 98 100.8) (end 98 100.199012) (width 0.1524) (layer F.Cu) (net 3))
 (segment (start 98.12447 101.660004) (end 98.492237 101.292237) (width 0.1524) (layer F.Cu) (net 3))
 (segment (start 98.492237 101.292237) (end 98.784474 101) (width 0.1524) (layer F.Cu) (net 3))
 (segment (start 101.95 99.75) (end 102 99.7) (width 0.1524) (layer F.Cu) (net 3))
 (segment (start 102 99.7) (end 102 98.464466) (width 0.1524) (layer F.Cu) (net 3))
 (segment (start 101.5 99.75) (end 101.95 99.75) (width 0.1524) (layer F.Cu) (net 3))
 (segment (start 102 100) (end 102 99.7) (width 0.1524) (layer F.Cu) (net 3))
 (segment (start 99.8476 102.5) (end 99.5 102.5) (width 0.1524) (layer F.Cu) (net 3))
 (segment (start 99.5 102.5) (end 99.5 101.5) (width 0.1524) (layer F.Cu) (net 3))
 (segment (start 99.5 101.5) (end 99.8476 101.5) (width 0.1524) (layer F.Cu) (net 3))
 (segment (start 99.5 101.5) (end 99.5 101) (width 0.1524) (layer F.Cu) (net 3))
 (segment (start 99.5 101) (end 99 101) (width 0.1524) (layer F.Cu) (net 3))
 (segment (start 99.8 101) (end 99.5 101) (width 0.1524) (layer F.Cu) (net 3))
 (segment (start 100 99.5) (end 100 100.5) (width 0.1524) (layer F.Cu) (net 2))
 (segment (start 100.32 94) (end 101 94) (width 0.1524) (layer B.Cu) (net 2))
 (via (at 101 94) (size 0.508) (drill 0.254) (layers F.Cu B.Cu) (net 2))
 (segment (start 101 94.5) (end 101 94) (width 0.1524) (layer F.Cu) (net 2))
 (segment (start 99.5 96) (end 101 94.5) (width 0.1524) (layer F.Cu) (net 2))
 (segment (start 100 99.5) (end 99.5 99) (width 0.1524) (layer F.Cu) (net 2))
 (segment (start 99.8476 98.5) (end 99.5 98.5) (width 0.1524) (layer F.Cu) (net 2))
 (segment (start 99.5 99) (end 99.5 98.5) (width 0.1524) (layer F.Cu) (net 2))
 (segment (start 99.8476 97.5) (end 99.5 97.5) (width 0.1524) (layer F.Cu) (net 2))
 (segment (start 99.5 97.5) (end 99.5 96) (width 0.1524) (layer F.Cu) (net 2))
 (segment (start 99.5 98.5) (end 99.5 97.5) (width 0.1524) (layer F.Cu) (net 2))
 (segment (start 101.25 100.5) (end 101.5 100.25) (width 0.1524) (layer F.Cu) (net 5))
 (segment (start 100.5 100.5) (end 101.25 100.5) (width 0.1524) (layer F.Cu) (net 5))
 (segment (start 99.68 94) (end 99 94) (width 0.1524) (layer B.Cu) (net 7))
 (via (at 99 94) (size 0.508) (drill 0.254) (layers F.Cu B.Cu) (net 7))
 (segment (start 99 98.28575) (end 99 95.8) (width 0.1524) (layer F.Cu) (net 7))
 (segment (start 99 95.8) (end 99 94) (width 0.1524) (layer F.Cu) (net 7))
 (segment (start 98.5 98.78575) (end 99 98.28575) (width 0.1524) (layer F.Cu) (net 7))
 (segment (start 98.5 99.75) (end 98.5 98.78575) (width 0.1524) (layer F.Cu) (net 7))
 (segment (start 98.75 100.25) (end 98.5 100.25) (width 0.1524) (layer F.Cu) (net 4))
 (segment (start 99.5 99.5) (end 98.75 100.25) (width 0.1524) (layer F.Cu) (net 4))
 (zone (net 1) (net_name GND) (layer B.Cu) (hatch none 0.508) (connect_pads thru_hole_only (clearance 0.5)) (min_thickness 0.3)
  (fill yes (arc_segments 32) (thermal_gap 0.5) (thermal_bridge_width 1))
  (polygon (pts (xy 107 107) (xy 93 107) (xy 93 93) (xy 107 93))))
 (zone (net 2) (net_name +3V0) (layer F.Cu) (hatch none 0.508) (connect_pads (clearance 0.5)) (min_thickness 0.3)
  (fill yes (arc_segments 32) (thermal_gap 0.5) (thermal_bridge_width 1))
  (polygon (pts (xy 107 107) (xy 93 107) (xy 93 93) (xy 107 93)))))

